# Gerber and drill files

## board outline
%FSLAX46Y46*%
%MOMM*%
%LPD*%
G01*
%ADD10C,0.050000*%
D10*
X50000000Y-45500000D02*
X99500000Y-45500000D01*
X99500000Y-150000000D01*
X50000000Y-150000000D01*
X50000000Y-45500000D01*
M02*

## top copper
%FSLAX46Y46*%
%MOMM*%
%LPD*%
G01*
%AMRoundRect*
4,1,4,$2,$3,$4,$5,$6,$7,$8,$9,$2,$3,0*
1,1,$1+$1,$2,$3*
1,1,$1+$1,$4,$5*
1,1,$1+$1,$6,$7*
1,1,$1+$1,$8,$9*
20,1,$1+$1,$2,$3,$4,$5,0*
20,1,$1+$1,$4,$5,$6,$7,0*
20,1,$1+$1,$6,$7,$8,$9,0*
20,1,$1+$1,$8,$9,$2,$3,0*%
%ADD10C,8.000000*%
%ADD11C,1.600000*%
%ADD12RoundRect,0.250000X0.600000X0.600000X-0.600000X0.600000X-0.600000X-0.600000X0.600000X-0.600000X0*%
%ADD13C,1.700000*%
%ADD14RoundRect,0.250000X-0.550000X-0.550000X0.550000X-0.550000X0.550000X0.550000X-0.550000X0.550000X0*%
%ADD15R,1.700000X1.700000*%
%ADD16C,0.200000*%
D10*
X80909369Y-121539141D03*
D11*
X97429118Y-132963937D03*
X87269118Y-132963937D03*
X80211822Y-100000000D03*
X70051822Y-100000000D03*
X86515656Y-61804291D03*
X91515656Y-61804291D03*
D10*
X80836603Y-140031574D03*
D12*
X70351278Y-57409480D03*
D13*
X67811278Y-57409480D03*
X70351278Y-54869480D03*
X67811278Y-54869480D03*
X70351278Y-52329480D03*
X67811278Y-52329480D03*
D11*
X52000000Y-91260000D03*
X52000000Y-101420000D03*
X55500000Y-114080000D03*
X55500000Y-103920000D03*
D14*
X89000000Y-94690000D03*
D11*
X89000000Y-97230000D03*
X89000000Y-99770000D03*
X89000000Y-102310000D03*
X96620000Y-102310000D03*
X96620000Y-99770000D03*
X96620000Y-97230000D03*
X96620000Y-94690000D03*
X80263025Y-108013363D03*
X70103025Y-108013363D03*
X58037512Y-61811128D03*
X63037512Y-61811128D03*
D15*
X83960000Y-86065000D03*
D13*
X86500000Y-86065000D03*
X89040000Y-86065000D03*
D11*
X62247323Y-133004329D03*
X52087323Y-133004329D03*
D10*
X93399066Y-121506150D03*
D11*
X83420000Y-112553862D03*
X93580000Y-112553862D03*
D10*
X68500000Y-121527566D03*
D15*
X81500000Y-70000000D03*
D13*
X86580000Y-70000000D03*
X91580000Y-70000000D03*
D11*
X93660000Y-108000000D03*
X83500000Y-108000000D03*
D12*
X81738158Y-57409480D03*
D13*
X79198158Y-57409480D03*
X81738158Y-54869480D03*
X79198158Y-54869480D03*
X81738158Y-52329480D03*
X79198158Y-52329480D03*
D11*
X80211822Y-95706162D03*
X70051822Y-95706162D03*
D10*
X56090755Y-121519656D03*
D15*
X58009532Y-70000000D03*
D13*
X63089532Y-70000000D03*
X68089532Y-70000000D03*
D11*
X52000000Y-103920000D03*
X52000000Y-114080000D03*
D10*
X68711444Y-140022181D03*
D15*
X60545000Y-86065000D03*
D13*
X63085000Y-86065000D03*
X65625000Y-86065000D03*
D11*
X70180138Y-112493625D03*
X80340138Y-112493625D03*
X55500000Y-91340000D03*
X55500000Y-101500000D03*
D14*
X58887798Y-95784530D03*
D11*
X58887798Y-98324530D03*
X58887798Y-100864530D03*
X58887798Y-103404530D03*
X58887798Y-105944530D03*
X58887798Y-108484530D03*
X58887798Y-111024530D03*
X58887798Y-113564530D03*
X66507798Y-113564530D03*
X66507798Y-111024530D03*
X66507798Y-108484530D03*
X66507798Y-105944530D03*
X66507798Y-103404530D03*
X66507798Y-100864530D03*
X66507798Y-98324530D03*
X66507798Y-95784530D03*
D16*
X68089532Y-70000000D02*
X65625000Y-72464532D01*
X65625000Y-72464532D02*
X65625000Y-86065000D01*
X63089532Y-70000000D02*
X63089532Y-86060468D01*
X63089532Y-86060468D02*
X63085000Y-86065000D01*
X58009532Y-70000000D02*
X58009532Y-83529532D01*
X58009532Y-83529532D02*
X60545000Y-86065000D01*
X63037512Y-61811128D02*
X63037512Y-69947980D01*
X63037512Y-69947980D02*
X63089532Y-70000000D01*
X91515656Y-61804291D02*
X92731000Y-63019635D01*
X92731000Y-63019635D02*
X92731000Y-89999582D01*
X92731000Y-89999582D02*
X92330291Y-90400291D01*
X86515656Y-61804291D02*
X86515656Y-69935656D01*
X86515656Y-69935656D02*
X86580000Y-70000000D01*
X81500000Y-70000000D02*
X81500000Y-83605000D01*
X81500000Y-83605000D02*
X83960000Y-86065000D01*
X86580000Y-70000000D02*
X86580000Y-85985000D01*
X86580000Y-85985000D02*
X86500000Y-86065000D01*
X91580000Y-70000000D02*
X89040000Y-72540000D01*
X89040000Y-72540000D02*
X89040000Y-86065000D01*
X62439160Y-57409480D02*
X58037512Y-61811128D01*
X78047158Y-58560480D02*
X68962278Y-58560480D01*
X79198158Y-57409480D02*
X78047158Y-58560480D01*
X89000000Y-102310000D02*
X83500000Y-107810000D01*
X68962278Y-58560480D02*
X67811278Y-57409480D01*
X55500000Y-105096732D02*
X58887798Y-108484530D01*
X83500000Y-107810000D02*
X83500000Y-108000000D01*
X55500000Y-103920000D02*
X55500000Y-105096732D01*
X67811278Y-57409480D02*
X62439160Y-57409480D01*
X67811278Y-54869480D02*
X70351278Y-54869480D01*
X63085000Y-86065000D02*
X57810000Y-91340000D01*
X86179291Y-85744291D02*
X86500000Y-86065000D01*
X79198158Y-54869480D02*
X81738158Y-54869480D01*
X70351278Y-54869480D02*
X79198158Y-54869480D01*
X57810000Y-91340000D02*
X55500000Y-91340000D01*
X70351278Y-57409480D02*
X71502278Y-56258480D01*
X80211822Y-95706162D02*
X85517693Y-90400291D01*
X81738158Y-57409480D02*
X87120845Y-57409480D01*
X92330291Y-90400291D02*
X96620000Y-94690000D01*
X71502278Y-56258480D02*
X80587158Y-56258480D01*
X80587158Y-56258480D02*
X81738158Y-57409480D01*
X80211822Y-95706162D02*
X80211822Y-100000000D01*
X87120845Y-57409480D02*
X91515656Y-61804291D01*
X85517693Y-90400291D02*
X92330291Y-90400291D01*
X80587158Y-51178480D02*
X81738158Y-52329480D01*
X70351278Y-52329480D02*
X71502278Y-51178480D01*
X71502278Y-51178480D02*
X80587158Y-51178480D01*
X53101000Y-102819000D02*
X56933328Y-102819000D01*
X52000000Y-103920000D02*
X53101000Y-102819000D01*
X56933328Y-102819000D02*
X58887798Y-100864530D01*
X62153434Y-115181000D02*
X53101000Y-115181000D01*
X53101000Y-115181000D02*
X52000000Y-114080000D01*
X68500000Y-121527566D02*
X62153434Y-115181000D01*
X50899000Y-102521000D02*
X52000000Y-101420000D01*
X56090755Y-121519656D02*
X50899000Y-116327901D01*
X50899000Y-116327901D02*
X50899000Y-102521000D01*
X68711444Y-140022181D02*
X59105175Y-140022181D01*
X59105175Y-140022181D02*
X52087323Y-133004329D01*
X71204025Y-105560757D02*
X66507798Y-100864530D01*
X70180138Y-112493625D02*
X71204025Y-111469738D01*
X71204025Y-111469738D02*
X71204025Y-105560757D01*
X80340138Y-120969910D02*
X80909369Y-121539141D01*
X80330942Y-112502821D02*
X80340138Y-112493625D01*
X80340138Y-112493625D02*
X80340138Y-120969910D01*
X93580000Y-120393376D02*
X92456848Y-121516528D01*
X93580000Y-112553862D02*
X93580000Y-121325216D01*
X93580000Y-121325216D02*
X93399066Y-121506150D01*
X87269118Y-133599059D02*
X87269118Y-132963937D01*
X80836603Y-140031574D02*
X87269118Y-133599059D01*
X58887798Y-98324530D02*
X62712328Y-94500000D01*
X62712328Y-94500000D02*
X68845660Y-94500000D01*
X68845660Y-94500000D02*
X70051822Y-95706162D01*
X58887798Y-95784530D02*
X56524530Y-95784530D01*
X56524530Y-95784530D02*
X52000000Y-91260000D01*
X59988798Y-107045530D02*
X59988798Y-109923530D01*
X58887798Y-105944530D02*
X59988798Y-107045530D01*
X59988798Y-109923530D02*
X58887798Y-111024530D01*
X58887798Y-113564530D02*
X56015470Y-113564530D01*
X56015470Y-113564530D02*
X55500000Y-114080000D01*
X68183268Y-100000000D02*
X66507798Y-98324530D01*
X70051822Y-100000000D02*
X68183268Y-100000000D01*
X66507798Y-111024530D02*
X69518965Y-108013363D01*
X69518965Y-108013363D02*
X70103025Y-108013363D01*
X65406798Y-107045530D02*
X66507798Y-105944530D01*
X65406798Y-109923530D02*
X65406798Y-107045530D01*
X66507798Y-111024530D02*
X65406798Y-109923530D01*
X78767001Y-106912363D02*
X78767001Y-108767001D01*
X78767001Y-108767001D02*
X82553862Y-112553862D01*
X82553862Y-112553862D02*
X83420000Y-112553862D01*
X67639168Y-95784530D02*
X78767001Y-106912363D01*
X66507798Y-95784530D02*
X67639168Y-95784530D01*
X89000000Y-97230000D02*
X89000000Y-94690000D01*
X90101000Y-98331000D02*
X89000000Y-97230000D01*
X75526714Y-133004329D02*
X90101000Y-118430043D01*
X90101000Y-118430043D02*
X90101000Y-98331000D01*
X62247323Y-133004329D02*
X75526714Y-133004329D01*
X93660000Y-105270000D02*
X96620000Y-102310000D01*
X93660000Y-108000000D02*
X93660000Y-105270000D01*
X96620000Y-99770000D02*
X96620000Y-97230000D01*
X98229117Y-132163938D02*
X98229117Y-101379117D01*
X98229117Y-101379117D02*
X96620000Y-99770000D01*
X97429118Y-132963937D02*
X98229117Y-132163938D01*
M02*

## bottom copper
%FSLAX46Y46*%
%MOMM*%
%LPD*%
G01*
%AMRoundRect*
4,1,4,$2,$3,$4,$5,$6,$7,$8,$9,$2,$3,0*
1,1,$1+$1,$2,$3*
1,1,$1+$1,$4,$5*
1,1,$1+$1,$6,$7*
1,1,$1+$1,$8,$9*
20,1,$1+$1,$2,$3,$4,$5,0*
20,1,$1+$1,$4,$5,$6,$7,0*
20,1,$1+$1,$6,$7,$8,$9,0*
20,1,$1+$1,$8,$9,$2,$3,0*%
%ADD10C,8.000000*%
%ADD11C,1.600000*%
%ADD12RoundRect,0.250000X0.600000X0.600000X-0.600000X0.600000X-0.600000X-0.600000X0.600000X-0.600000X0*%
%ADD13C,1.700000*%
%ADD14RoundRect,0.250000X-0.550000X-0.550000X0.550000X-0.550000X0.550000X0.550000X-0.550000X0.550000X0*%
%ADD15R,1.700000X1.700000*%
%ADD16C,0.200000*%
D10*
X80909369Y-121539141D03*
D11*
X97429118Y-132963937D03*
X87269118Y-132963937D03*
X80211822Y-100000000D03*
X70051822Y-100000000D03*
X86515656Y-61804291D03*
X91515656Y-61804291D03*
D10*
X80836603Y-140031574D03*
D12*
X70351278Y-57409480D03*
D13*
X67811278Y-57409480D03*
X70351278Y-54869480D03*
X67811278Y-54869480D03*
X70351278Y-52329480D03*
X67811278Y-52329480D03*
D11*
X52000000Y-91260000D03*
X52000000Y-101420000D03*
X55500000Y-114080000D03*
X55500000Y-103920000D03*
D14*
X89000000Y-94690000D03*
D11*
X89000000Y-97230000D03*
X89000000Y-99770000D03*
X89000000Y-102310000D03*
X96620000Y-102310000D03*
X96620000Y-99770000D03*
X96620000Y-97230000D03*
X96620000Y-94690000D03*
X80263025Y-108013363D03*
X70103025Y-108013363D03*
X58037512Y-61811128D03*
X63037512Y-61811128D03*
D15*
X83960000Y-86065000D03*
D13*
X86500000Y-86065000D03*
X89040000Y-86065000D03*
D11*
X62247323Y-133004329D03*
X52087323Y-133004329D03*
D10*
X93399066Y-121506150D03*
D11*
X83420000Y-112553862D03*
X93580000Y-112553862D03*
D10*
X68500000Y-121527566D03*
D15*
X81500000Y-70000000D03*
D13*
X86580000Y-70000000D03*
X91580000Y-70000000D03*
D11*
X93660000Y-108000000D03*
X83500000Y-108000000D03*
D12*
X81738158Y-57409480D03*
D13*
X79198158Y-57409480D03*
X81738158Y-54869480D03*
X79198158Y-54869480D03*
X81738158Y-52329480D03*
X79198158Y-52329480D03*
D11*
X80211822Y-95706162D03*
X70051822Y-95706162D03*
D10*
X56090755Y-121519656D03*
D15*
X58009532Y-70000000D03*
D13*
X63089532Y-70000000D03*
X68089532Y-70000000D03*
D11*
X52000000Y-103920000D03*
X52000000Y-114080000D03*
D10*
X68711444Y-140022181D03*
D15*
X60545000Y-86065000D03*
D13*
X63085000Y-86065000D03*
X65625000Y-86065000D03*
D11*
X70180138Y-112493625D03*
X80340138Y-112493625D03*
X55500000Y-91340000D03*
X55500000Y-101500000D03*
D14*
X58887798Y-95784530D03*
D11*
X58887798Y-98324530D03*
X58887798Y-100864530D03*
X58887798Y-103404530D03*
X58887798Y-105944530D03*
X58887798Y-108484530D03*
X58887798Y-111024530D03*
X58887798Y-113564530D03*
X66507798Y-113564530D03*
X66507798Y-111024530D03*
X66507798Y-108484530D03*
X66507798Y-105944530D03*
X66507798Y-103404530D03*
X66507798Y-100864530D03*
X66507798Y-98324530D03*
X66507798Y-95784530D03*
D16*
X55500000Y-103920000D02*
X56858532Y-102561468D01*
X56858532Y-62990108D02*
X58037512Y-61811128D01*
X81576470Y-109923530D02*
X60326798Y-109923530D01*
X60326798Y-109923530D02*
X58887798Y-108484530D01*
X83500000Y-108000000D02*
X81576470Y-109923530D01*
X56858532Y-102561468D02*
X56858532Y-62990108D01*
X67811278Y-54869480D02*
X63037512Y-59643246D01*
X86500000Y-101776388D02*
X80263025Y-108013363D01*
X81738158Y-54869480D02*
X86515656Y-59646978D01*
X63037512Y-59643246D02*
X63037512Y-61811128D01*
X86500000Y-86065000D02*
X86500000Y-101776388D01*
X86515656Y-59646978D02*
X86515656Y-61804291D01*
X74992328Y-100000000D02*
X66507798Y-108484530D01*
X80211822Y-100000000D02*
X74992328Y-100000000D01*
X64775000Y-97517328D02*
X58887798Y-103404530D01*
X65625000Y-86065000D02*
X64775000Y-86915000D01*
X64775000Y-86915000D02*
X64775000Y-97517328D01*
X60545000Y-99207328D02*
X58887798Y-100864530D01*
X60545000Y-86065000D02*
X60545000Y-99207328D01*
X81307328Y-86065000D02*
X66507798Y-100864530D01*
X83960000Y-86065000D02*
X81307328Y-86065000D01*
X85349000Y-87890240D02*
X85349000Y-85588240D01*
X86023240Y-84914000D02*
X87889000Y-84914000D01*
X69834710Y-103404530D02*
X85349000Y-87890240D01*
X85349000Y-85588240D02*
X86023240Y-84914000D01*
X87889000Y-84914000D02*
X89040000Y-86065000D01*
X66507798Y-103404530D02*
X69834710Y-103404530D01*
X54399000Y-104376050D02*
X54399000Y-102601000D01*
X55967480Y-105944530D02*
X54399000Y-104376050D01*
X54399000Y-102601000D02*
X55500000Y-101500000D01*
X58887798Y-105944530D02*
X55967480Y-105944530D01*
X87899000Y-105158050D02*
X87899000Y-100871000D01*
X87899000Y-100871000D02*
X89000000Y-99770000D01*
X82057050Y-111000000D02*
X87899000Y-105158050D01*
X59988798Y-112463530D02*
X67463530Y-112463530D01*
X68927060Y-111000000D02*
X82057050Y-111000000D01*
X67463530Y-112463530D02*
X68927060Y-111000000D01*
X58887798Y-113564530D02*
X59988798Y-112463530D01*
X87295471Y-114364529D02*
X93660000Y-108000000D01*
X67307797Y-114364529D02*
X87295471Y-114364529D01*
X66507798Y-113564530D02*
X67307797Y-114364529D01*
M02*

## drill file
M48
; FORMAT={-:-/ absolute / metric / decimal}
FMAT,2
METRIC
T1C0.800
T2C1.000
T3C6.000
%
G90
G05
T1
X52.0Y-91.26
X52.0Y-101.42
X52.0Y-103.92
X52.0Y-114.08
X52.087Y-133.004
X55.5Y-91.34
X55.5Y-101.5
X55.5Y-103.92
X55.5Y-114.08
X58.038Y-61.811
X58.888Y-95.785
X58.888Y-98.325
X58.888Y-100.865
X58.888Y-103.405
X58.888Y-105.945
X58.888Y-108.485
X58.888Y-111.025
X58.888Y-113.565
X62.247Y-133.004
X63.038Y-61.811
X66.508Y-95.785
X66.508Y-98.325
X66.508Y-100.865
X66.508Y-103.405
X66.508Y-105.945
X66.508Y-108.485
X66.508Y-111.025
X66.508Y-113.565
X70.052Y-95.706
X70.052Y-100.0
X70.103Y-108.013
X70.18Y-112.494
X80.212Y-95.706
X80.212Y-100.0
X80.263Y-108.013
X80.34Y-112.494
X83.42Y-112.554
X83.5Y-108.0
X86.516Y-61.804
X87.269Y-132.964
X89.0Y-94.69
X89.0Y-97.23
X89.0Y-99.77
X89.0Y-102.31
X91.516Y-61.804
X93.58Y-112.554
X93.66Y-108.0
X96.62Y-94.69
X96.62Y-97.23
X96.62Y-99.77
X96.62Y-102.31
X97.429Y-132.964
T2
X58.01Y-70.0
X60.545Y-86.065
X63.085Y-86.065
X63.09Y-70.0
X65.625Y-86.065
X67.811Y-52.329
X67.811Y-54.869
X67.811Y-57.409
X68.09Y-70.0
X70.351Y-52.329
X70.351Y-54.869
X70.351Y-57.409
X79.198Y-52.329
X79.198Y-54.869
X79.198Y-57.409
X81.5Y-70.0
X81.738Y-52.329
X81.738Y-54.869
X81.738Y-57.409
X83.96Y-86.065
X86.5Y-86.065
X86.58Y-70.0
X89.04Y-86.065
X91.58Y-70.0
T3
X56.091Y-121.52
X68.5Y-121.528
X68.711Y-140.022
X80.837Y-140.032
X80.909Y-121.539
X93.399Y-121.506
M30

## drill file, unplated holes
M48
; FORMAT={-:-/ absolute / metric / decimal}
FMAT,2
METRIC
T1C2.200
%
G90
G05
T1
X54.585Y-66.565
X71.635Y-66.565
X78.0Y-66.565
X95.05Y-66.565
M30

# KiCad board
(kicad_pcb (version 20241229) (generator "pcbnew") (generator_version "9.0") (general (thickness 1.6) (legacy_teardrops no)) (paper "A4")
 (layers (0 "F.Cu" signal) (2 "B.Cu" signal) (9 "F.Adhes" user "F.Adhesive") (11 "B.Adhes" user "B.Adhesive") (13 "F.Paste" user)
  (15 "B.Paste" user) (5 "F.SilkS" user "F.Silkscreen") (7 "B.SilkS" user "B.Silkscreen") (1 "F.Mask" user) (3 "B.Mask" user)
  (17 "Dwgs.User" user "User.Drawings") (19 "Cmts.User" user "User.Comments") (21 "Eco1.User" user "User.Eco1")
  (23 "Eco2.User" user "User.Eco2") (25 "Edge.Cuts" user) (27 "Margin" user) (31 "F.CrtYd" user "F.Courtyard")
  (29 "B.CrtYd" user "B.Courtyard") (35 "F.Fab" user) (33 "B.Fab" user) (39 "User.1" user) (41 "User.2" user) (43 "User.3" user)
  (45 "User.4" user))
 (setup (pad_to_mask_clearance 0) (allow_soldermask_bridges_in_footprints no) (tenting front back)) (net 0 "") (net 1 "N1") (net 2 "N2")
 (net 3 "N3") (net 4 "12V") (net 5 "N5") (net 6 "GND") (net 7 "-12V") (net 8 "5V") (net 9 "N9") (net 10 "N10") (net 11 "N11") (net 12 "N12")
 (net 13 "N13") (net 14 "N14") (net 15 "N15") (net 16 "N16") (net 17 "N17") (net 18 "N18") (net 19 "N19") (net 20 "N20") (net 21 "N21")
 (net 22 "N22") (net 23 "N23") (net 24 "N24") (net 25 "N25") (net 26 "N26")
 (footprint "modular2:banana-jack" (layer "F.Cu") (at 80.909369 121.514203)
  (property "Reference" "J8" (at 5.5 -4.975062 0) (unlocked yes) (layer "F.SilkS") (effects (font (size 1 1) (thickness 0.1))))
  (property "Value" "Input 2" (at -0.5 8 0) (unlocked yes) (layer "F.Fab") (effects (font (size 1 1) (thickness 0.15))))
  (pad "1" thru_hole circle (at 0 0.024938) (size 8 8) (drill 6) (layers "*.Cu" "*.Mask") (remove_unused_layers no) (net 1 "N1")))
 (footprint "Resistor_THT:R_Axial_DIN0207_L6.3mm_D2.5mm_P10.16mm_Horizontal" (layer "F.Cu") (at 97.429118 132.963937 180)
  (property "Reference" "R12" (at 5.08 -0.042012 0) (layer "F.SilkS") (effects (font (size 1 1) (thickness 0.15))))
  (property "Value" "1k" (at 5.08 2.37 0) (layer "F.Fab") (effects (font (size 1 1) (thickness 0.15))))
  (pad "1" thru_hole circle (at 0 0 180) (size 1.6 1.6) (drill 0.8) (layers "*.Cu" "*.Mask") (remove_unused_layers no) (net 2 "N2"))
  (pad "2" thru_hole circle (at 10.16 0 180) (size 1.6 1.6) (drill 0.8) (layers "*.Cu" "*.Mask") (remove_unused_layers no) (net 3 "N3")))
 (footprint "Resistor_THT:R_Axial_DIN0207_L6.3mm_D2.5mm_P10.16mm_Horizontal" (layer "F.Cu") (at 80.211822 100 180)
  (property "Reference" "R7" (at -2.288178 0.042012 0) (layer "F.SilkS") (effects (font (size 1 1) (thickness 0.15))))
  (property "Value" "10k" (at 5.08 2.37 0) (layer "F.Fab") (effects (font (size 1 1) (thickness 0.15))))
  (pad "1" thru_hole circle (at 0 0 180) (size 1.6 1.6) (drill 0.8) (layers "*.Cu" "*.Mask") (remove_unused_layers no) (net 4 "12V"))
  (pad "2" thru_hole circle (at 10.16 0 180) (size 1.6 1.6) (drill 0.8) (layers "*.Cu" "*.Mask") (remove_unused_layers no) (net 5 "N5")))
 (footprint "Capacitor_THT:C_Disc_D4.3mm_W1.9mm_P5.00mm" (layer "F.Cu") (at 86.515656 61.804291)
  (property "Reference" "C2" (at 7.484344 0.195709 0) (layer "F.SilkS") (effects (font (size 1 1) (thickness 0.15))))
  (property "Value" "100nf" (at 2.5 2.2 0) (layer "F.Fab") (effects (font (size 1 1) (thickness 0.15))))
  (pad "1" thru_hole circle (at 0 0) (size 1.6 1.6) (drill 0.8) (layers "*.Cu" "*.Mask") (remove_unused_layers no) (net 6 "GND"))
  (pad "2" thru_hole circle (at 5 0) (size 1.6 1.6) (drill 0.8) (layers "*.Cu" "*.Mask") (remove_unused_layers no) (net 4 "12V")))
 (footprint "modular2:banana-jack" (layer "F.Cu") (at 80.836603 140.006636)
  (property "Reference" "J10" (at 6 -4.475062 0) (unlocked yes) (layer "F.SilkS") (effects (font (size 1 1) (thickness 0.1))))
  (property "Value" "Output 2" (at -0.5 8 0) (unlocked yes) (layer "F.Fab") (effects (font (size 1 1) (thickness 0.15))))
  (pad "1" thru_hole circle (at 0 0.024938) (size 8 8) (drill 6) (layers "*.Cu" "*.Mask") (remove_unused_layers no) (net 3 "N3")))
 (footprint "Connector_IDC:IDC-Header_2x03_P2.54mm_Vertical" (layer "F.Cu") (at 70.351278 57.40948 180)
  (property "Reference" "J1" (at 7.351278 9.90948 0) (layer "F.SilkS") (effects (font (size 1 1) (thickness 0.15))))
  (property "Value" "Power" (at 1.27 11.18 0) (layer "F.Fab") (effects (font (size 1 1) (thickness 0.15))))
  (pad "1" thru_hole roundrect (at 0 0 180) (size 1.7 1.7) (drill 1) (layers "*.Cu" "*.Mask") (remove_unused_layers no)
   (roundrect_rratio 0.147059) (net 4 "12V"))
  (pad "2" thru_hole circle (at 2.54 0 180) (size 1.7 1.7) (drill 1) (layers "*.Cu" "*.Mask") (remove_unused_layers no) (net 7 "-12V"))
  (pad "3" thru_hole circle (at 0 2.54 180) (size 1.7 1.7) (drill 1) (layers "*.Cu" "*.Mask") (remove_unused_layers no) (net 6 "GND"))
  (pad "4" thru_hole circle (at 2.54 2.54 180) (size 1.7 1.7) (drill 1) (layers "*.Cu" "*.Mask") (remove_unused_layers no) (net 6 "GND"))
  (pad "5" thru_hole circle (at 0 5.08 180) (size 1.7 1.7) (drill 1) (layers "*.Cu" "*.Mask") (remove_unused_layers no) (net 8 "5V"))
  (pad "6" thru_hole circle (at 2.54 5.08 180) (size 1.7 1.7) (drill 1) (layers "*.Cu" "*.Mask") (remove_unused_layers no) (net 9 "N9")))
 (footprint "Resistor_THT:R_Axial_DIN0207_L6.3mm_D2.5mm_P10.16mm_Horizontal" (layer "F.Cu") (at 52 91.26 -90)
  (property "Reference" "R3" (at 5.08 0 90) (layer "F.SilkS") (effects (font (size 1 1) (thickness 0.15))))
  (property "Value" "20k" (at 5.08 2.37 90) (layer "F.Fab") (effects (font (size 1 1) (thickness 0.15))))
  (pad "1" thru_hole circle (at 0 0 270) (size 1.6 1.6) (drill 0.8) (layers "*.Cu" "*.Mask") (remove_unused_layers no) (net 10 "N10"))
  (pad "2" thru_hole circle (at 10.16 0 270) (size 1.6 1.6) (drill 0.8) (layers "*.Cu" "*.Mask") (remove_unused_layers no) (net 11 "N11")))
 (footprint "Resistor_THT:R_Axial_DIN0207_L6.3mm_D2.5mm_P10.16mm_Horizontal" (layer "F.Cu") (at 55.5 114.08 90)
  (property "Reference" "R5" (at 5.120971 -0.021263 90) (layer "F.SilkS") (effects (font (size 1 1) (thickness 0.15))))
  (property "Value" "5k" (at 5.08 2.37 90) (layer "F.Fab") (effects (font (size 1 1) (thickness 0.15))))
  (pad "1" thru_hole circle (at 0 0 90) (size 1.6 1.6) (drill 0.8) (layers "*.Cu" "*.Mask") (remove_unused_layers no) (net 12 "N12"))
  (pad "2" thru_hole circle (at 10.16 0 90) (size 1.6 1.6) (drill 0.8) (layers "*.Cu" "*.Mask") (remove_unused_layers no) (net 7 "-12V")))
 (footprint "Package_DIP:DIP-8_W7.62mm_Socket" (layer "F.Cu") (at 89 94.69)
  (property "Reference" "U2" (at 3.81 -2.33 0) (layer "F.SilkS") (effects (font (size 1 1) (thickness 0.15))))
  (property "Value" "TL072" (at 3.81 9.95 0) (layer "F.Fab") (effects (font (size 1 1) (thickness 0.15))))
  (pad "1" thru_hole roundrect (at 0 0) (size 1.6 1.6) (drill 0.8) (layers "*.Cu" "*.Mask") (remove_unused_layers no)
   (roundrect_rratio 0.15625) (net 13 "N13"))
  (pad "2" thru_hole circle (at 0 2.54) (size 1.6 1.6) (drill 0.8) (layers "*.Cu" "*.Mask") (remove_unused_layers no) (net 13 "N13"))
  (pad "3" thru_hole circle (at 0 5.08) (size 1.6 1.6) (drill 0.8) (layers "*.Cu" "*.Mask") (remove_unused_layers no) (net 12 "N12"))
  (pad "4" thru_hole circle (at 0 7.62) (size 1.6 1.6) (drill 0.8) (layers "*.Cu" "*.Mask") (remove_unused_layers no) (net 7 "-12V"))
  (pad "5" thru_hole circle (at 7.62 7.62) (size 1.6 1.6) (drill 0.8) (layers "*.Cu" "*.Mask") (remove_unused_layers no) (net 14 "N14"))
  (pad "6" thru_hole circle (at 7.62 5.08) (size 1.6 1.6) (drill 0.8) (layers "*.Cu" "*.Mask") (remove_unused_layers no) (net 2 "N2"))
  (pad "7" thru_hole circle (at 7.62 2.54) (size 1.6 1.6) (drill 0.8) (layers "*.Cu" "*.Mask") (remove_unused_layers no) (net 2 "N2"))
  (pad "8" thru_hole circle (at 7.62 0) (size 1.6 1.6) (drill 0.8) (layers "*.Cu" "*.Mask") (remove_unused_layers no) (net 4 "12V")))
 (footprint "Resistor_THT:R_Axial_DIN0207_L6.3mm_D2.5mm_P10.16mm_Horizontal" (layer "F.Cu") (at 80.263025 108.013363 180)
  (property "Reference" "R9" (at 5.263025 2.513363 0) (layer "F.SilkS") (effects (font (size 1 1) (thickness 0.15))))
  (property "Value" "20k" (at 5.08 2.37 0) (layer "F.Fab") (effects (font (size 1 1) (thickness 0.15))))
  (pad "1" thru_hole circle (at 0 0 180) (size 1.6 1.6) (drill 0.8) (layers "*.Cu" "*.Mask") (remove_unused_layers no) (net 6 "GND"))
  (pad "2" thru_hole circle (at 10.16 0 180) (size 1.6 1.6) (drill 0.8) (layers "*.Cu" "*.Mask") (remove_unused_layers no) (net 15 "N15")))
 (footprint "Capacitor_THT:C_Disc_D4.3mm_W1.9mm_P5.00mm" (layer "F.Cu") (at 58.037512 61.811128)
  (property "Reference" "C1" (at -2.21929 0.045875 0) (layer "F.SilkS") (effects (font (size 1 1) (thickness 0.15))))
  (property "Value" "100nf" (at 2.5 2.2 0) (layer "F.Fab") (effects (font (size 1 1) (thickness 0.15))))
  (pad "1" thru_hole circle (at 0 0) (size 1.6 1.6) (drill 0.8) (layers "*.Cu" "*.Mask") (remove_unused_layers no) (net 7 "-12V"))
  (pad "2" thru_hole circle (at 5 0) (size 1.6 1.6) (drill 0.8) (layers "*.Cu" "*.Mask") (remove_unused_layers no) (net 6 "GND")))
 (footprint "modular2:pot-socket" (layer "F.Cu") (at 85.5 78.065)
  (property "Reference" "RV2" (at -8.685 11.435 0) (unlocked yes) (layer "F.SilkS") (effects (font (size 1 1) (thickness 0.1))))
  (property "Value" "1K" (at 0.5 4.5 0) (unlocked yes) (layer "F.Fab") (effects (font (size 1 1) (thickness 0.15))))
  (pad "" np_thru_hole circle (at -7.5 -11.5) (size 2.2 2.2) (drill 2.2) (layers "*.Cu" "*.Mask"))
  (pad "" np_thru_hole circle (at 9.55 -11.5) (size 2.2 2.2) (drill 2.2) (layers "*.Cu" "*.Mask"))
  (pad "1" thru_hole rect (at -1.54 8 90) (size 1.7 1.7) (drill 1) (layers "*.Cu" "*.Mask") (remove_unused_layers no) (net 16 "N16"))
  (pad "2" thru_hole circle (at 1 8 90) (size 1.7 1.7) (drill 1) (layers "*.Cu" "*.Mask") (remove_unused_layers no) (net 6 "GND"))
  (pad "3" thru_hole circle (at 3.54 8 90) (size 1.7 1.7) (drill 1) (layers "*.Cu" "*.Mask") (remove_unused_layers no) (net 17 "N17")))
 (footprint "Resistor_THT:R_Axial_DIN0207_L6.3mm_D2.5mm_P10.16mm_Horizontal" (layer "F.Cu") (at 62.247323 133.004329 180)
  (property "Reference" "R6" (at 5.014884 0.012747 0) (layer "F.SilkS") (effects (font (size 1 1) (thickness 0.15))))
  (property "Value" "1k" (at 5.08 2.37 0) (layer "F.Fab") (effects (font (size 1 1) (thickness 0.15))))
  (pad "1" thru_hole circle (at 0 0 180) (size 1.6 1.6) (drill 0.8) (layers "*.Cu" "*.Mask") (remove_unused_layers no) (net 13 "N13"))
  (pad "2" thru_hole circle (at 10.16 0 180) (size 1.6 1.6) (drill 0.8) (layers "*.Cu" "*.Mask") (remove_unused_layers no) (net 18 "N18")))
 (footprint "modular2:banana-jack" (layer "F.Cu") (at 93.399066 121.481212)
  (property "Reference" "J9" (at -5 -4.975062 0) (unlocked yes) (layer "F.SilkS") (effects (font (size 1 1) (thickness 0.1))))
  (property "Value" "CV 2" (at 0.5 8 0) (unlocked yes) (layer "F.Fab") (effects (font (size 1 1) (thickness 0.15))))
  (pad "1" thru_hole circle (at 0 0.024938) (size 8 8) (drill 6) (layers "*.Cu" "*.Mask") (remove_unused_layers no) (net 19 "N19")))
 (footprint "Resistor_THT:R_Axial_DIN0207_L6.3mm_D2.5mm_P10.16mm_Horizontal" (layer "F.Cu") (at 83.42 112.553862)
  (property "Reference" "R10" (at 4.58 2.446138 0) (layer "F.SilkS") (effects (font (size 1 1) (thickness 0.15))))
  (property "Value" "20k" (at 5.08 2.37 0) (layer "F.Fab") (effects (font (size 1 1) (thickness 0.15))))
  (pad "1" thru_hole circle (at 0 0) (size 1.6 1.6) (drill 0.8) (layers "*.Cu" "*.Mask") (remove_unused_layers no) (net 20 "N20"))
  (pad "2" thru_hole circle (at 10.16 0) (size 1.6 1.6) (drill 0.8) (layers "*.Cu" "*.Mask") (remove_unused_layers no) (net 19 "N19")))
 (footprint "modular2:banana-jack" (layer "F.Cu") (at 68.5 121.502628)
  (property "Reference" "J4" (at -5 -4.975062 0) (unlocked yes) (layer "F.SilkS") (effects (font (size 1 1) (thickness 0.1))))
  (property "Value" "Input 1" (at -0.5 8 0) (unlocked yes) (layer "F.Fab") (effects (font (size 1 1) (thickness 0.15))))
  (pad "1" thru_hole circle (at 0 0.024938) (size 8 8) (drill 6) (layers "*.Cu" "*.Mask") (remove_unused_layers no) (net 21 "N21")))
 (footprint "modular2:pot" (layer "F.Cu") (at 86.58 73)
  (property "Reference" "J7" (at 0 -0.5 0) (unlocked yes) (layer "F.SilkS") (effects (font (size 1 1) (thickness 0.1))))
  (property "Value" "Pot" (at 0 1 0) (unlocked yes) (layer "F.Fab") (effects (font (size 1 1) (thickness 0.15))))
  (pad "1" thru_hole rect (at -5.08 -3 90) (size 1.7 1.7) (drill 1) (layers "*.Cu" "*.Mask") (remove_unused_layers no) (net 16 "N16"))
  (pad "2" thru_hole circle (at 0 -3 90) (size 1.7 1.7) (drill 1) (layers "*.Cu" "*.Mask") (remove_unused_layers no) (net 6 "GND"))
  (pad "3" thru_hole circle (at 5 -3 90) (size 1.7 1.7) (drill 1) (layers "*.Cu" "*.Mask") (remove_unused_layers no) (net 17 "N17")))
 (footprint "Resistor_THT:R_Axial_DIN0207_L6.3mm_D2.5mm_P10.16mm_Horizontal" (layer "F.Cu") (at 93.66 108 180)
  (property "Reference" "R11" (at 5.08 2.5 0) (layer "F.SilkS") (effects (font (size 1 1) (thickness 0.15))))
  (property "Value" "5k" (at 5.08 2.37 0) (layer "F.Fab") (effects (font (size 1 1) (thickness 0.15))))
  (pad "1" thru_hole circle (at 0 0 180) (size 1.6 1.6) (drill 0.8) (layers "*.Cu" "*.Mask") (remove_unused_layers no) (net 14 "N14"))
  (pad "2" thru_hole circle (at 10.16 0 180) (size 1.6 1.6) (drill 0.8) (layers "*.Cu" "*.Mask") (remove_unused_layers no) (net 7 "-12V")))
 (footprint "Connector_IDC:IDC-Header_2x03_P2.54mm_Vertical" (layer "F.Cu") (at 81.738158 57.40948 180)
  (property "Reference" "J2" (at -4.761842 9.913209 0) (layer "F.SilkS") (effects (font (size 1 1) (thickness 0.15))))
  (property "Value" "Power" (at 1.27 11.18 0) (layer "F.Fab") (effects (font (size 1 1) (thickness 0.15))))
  (pad "1" thru_hole roundrect (at 0 0 180) (size 1.7 1.7) (drill 1) (layers "*.Cu" "*.Mask") (remove_unused_layers no)
   (roundrect_rratio 0.147059) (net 4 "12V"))
  (pad "2" thru_hole circle (at 2.54 0 180) (size 1.7 1.7) (drill 1) (layers "*.Cu" "*.Mask") (remove_unused_layers no) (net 7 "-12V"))
  (pad "3" thru_hole circle (at 0 2.54 180) (size 1.7 1.7) (drill 1) (layers "*.Cu" "*.Mask") (remove_unused_layers no) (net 6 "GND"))
  (pad "4" thru_hole circle (at 2.54 2.54 180) (size 1.7 1.7) (drill 1) (layers "*.Cu" "*.Mask") (remove_unused_layers no) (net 6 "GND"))
  (pad "5" thru_hole circle (at 0 5.08 180) (size 1.7 1.7) (drill 1) (layers "*.Cu" "*.Mask") (remove_unused_layers no) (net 8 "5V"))
  (pad "6" thru_hole circle (at 2.54 5.08 180) (size 1.7 1.7) (drill 1) (layers "*.Cu" "*.Mask") (remove_unused_layers no) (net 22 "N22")))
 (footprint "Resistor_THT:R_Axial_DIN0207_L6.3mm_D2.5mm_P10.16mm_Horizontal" (layer "F.Cu") (at 80.211822 95.706162 180)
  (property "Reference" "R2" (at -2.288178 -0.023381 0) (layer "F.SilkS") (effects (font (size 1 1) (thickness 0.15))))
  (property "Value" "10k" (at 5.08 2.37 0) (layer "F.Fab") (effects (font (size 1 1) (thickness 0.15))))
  (pad "1" thru_hole circle (at 0 0 180) (size 1.6 1.6) (drill 0.8) (layers "*.Cu" "*.Mask") (remove_unused_layers no) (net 4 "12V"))
  (pad "2" thru_hole circle (at 10.16 0 180) (size 1.6 1.6) (drill 0.8) (layers "*.Cu" "*.Mask") (remove_unused_layers no) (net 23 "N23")))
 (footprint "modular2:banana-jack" (layer "F.Cu") (at 56.090755 121.494718)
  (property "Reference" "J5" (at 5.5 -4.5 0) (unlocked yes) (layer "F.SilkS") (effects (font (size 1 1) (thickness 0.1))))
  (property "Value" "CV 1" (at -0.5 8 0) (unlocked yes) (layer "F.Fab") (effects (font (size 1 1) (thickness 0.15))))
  (pad "1" thru_hole circle (at 0 0.024938) (size 8 8) (drill 6) (layers "*.Cu" "*.Mask") (remove_unused_layers no) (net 11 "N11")))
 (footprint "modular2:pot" (layer "F.Cu") (at 63.089532 73)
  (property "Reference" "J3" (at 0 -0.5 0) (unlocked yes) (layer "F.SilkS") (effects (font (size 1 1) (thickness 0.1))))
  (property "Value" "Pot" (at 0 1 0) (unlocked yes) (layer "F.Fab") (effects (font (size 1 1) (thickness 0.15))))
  (pad "1" thru_hole rect (at -5.08 -3 90) (size 1.7 1.7) (drill 1) (layers "*.Cu" "*.Mask") (remove_unused_layers no) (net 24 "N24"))
  (pad "2" thru_hole circle (at 0 -3 90) (size 1.7 1.7) (drill 1) (layers "*.Cu" "*.Mask") (remove_unused_layers no) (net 6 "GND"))
  (pad "3" thru_hole circle (at 5 -3 90) (size 1.7 1.7) (drill 1) (layers "*.Cu" "*.Mask") (remove_unused_layers no) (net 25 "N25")))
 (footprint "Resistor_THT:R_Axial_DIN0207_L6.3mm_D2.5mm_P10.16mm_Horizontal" (layer "F.Cu") (at 52 103.92 -90)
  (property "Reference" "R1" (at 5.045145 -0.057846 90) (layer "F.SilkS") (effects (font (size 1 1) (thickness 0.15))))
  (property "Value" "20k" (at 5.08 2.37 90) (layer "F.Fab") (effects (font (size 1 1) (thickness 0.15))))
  (pad "1" thru_hole circle (at 0 0 270) (size 1.6 1.6) (drill 0.8) (layers "*.Cu" "*.Mask") (remove_unused_layers no) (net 24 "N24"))
  (pad "2" thru_hole circle (at 10.16 0 270) (size 1.6 1.6) (drill 0.8) (layers "*.Cu" "*.Mask") (remove_unused_layers no) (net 21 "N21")))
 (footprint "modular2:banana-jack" (layer "F.Cu") (at 68.711444 139.997243)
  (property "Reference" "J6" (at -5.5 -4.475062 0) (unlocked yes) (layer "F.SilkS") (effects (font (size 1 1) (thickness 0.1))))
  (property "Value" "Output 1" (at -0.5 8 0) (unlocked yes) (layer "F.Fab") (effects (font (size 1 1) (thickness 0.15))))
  (pad "1" thru_hole circle (at 0 0.024938) (size 8 8) (drill 6) (layers "*.Cu" "*.Mask") (remove_unused_layers no) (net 18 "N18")))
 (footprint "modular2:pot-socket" (layer "F.Cu") (at 62.085 78.065)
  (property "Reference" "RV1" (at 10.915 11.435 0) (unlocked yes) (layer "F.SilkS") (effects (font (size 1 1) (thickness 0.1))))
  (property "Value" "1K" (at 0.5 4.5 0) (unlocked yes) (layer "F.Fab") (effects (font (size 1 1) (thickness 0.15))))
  (pad "" np_thru_hole circle (at -7.5 -11.5) (size 2.2 2.2) (drill 2.2) (layers "*.Cu" "*.Mask"))
  (pad "" np_thru_hole circle (at 9.55 -11.5) (size 2.2 2.2) (drill 2.2) (layers "*.Cu" "*.Mask"))
  (pad "1" thru_hole rect (at -1.54 8 90) (size 1.7 1.7) (drill 1) (layers "*.Cu" "*.Mask") (remove_unused_layers no) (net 24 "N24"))
  (pad "2" thru_hole circle (at 1 8 90) (size 1.7 1.7) (drill 1) (layers "*.Cu" "*.Mask") (remove_unused_layers no) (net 6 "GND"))
  (pad "3" thru_hole circle (at 3.54 8 90) (size 1.7 1.7) (drill 1) (layers "*.Cu" "*.Mask") (remove_unused_layers no) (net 25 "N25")))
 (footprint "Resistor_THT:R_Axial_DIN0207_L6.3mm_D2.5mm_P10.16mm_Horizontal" (layer "F.Cu") (at 70.180138 112.493625)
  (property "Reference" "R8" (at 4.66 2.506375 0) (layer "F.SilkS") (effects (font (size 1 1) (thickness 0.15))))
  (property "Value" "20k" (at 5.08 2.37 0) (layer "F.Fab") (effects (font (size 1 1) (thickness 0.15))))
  (pad "1" thru_hole circle (at 0 0) (size 1.6 1.6) (drill 0.8) (layers "*.Cu" "*.Mask") (remove_unused_layers no) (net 16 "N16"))
  (pad "2" thru_hole circle (at 10.16 0) (size 1.6 1.6) (drill 0.8) (layers "*.Cu" "*.Mask") (remove_unused_layers no) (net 1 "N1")))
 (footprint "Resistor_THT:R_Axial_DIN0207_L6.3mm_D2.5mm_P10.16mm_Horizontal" (layer "F.Cu") (at 55.5 91.34 -90)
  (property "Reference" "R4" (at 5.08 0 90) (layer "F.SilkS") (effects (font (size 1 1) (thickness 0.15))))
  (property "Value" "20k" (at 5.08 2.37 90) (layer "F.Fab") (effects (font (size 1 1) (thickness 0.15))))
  (pad "1" thru_hole circle (at 0 0 270) (size 1.6 1.6) (drill 0.8) (layers "*.Cu" "*.Mask") (remove_unused_layers no) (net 6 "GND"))
  (pad "2" thru_hole circle (at 10.16 0 270) (size 1.6 1.6) (drill 0.8) (layers "*.Cu" "*.Mask") (remove_unused_layers no) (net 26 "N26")))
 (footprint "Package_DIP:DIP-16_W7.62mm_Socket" (layer "F.Cu") (at 58.887798 95.78453)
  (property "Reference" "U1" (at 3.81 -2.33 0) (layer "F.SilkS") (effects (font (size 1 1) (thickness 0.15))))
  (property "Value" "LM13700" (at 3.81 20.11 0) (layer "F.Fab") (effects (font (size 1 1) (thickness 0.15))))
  (pad "1" thru_hole roundrect (at 0 0) (size 1.6 1.6) (drill 0.8) (layers "*.Cu" "*.Mask") (remove_unused_layers no)
   (roundrect_rratio 0.15625) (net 10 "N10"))
  (pad "2" thru_hole circle (at 0 2.54) (size 1.6 1.6) (drill 0.8) (layers "*.Cu" "*.Mask") (remove_unused_layers no) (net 23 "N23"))
  (pad "3" thru_hole circle (at 0 5.08) (size 1.6 1.6) (drill 0.8) (layers "*.Cu" "*.Mask") (remove_unused_layers no) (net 24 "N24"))
  (pad "4" thru_hole circle (at 0 7.62) (size 1.6 1.6) (drill 0.8) (layers "*.Cu" "*.Mask") (remove_unused_layers no) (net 25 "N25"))
  (pad "5" thru_hole circle (at 0 10.16) (size 1.6 1.6) (drill 0.8) (layers "*.Cu" "*.Mask") (remove_unused_layers no) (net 26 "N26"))
  (pad "6" thru_hole circle (at 0 12.7) (size 1.6 1.6) (drill 0.8) (layers "*.Cu" "*.Mask") (remove_unused_layers no) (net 7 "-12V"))
  (pad "7" thru_hole circle (at 0 15.24) (size 1.6 1.6) (drill 0.8) (layers "*.Cu" "*.Mask") (remove_unused_layers no) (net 26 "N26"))
  (pad "8" thru_hole circle (at 0 17.78) (size 1.6 1.6) (drill 0.8) (layers "*.Cu" "*.Mask") (remove_unused_layers no) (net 12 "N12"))
  (pad "9" thru_hole circle (at 7.62 17.78) (size 1.6 1.6) (drill 0.8) (layers "*.Cu" "*.Mask") (remove_unused_layers no) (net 14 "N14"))
  (pad "10" thru_hole circle (at 7.62 15.24) (size 1.6 1.6) (drill 0.8) (layers "*.Cu" "*.Mask") (remove_unused_layers no) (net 15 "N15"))
  (pad "11" thru_hole circle (at 7.62 12.7) (size 1.6 1.6) (drill 0.8) (layers "*.Cu" "*.Mask") (remove_unused_layers no) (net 4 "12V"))
  (pad "12" thru_hole circle (at 7.62 10.16) (size 1.6 1.6) (drill 0.8) (layers "*.Cu" "*.Mask") (remove_unused_layers no) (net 15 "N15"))
  (pad "13" thru_hole circle (at 7.62 7.62) (size 1.6 1.6) (drill 0.8) (layers "*.Cu" "*.Mask") (remove_unused_layers no) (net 17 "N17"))
  (pad "14" thru_hole circle (at 7.62 5.08) (size 1.6 1.6) (drill 0.8) (layers "*.Cu" "*.Mask") (remove_unused_layers no) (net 16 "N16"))
  (pad "15" thru_hole circle (at 7.62 2.54) (size 1.6 1.6) (drill 0.8) (layers "*.Cu" "*.Mask") (remove_unused_layers no) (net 5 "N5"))
  (pad "16" thru_hole circle (at 7.62 0) (size 1.6 1.6) (drill 0.8) (layers "*.Cu" "*.Mask") (remove_unused_layers no) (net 20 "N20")))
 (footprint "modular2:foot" (layer "B.Cu") (at 56.59315 142.948114 180)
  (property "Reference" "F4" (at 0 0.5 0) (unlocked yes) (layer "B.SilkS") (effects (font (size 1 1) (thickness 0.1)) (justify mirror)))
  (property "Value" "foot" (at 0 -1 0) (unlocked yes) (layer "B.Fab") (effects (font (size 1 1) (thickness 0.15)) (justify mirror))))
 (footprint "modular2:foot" (layer "B.Cu") (at 92.94531 142.941798 180)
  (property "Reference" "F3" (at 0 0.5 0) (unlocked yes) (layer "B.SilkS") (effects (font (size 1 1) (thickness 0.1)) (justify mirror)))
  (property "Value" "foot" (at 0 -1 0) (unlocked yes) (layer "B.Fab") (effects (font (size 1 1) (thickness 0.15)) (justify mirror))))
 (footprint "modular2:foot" (layer "B.Cu") (at 56.600318 52.099806 180)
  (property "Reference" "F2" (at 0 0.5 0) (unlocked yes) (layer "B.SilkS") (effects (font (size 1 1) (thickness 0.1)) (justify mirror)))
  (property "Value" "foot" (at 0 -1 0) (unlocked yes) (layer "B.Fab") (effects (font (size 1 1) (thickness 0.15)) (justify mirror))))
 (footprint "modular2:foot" (layer "B.Cu") (at 92.943332 52.071217 180)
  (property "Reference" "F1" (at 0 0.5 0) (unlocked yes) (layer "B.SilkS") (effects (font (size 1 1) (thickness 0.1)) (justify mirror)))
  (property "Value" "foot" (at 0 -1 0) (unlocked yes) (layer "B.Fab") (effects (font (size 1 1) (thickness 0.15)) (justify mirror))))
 (gr_rect (start 50 45.5) (end 99.5 150) (stroke (width 0.05) (type default)) (fill no) (layer "Edge.Cuts"))
 (segment (start 62.43916 57.40948) (end 58.037512 61.811128) (width 0.2) (layer "F.Cu") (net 7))
 (segment (start 78.047158 58.56048) (end 68.962278 58.56048) (width 0.2) (layer "F.Cu") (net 7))
 (segment (start 79.198158 57.40948) (end 78.047158 58.56048) (width 0.2) (layer "F.Cu") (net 7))
 (segment (start 89 102.31) (end 83.5 107.81) (width 0.2) (layer "F.Cu") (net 7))
 (segment (start 68.962278 58.56048) (end 67.811278 57.40948) (width 0.2) (layer "F.Cu") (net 7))
 (segment (start 55.5 105.096732) (end 58.887798 108.48453) (width 0.2) (layer "F.Cu") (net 7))
 (segment (start 83.5 107.81) (end 83.5 108) (width 0.2) (layer "F.Cu") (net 7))
 (segment (start 55.5 103.92) (end 55.5 105.096732) (width 0.2) (layer "F.Cu") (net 7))
 (segment (start 67.811278 57.40948) (end 62.43916 57.40948) (width 0.2) (layer "F.Cu") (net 7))
 (segment (start 55.5 103.92) (end 56.858532 102.561468) (width 0.2) (layer "B.Cu") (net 7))
 (segment (start 56.858532 62.990108) (end 58.037512 61.811128) (width 0.2) (layer "B.Cu") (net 7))
 (segment (start 81.57647 109.92353) (end 60.326798 109.92353) (width 0.2) (layer "B.Cu") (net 7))
 (segment (start 60.326798 109.92353) (end 58.887798 108.48453) (width 0.2) (layer "B.Cu") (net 7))
 (segment (start 83.5 108) (end 81.57647 109.92353) (width 0.2) (layer "B.Cu") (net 7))
 (segment (start 56.858532 102.561468) (end 56.858532 62.990108) (width 0.2) (layer "B.Cu") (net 7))
 (segment (start 67.811278 54.86948) (end 70.351278 54.86948) (width 0.2) (layer "F.Cu") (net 6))
 (segment (start 63.089532 86.060468) (end 63.085 86.065) (width 0.2) (layer "F.Cu") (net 6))
 (segment (start 63.037512 61.811128) (end 63.037512 69.94798) (width 0.2) (layer "F.Cu") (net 6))
 (segment (start 86.58 85.985) (end 86.5 86.065) (width 0.2) (layer "F.Cu") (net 6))
 (segment (start 63.085 86.065) (end 57.81 91.34) (width 0.2) (layer "F.Cu") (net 6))
 (segment (start 86.179291 85.744291) (end 86.5 86.065) (width 0.2) (layer "F.Cu") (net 6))
 (segment (start 79.198158 54.86948) (end 81.738158 54.86948) (width 0.2) (layer "F.Cu") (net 6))
 (segment (start 63.037512 69.94798) (end 63.089532 70) (width 0.2) (layer "F.Cu") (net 6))
 (segment (start 70.351278 54.86948) (end 79.198158 54.86948) (width 0.2) (layer "F.Cu") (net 6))
 (segment (start 86.515656 69.935656) (end 86.58 70) (width 0.2) (layer "F.Cu") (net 6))
 (segment (start 57.81 91.34) (end 55.5 91.34) (width 0.2) (layer "F.Cu") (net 6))
 (segment (start 86.58 70) (end 86.58 85.985) (width 0.2) (layer "F.Cu") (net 6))
 (segment (start 63.089532 70) (end 63.089532 86.060468) (width 0.2) (layer "F.Cu") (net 6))
 (segment (start 86.515656 61.804291) (end 86.515656 69.935656) (width 0.2) (layer "F.Cu") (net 6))
 (segment (start 67.811278 54.86948) (end 63.037512 59.643246) (width 0.2) (layer "B.Cu") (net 6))
 (segment (start 86.5 101.776388) (end 80.263025 108.013363) (width 0.2) (layer "B.Cu") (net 6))
 (segment (start 81.738158 54.86948) (end 86.515656 59.646978) (width 0.2) (layer "B.Cu") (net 6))
 (segment (start 63.037512 59.643246) (end 63.037512 61.811128) (width 0.2) (layer "B.Cu") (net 6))
 (segment (start 86.5 86.065) (end 86.5 101.776388) (width 0.2) (layer "B.Cu") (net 6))
 (segment (start 86.515656 59.646978) (end 86.515656 61.804291) (width 0.2) (layer "B.Cu") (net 6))
 (segment (start 70.351278 57.40948) (end 71.502278 56.25848) (width 0.2) (layer "F.Cu") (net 4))
 (segment (start 80.211822 95.706162) (end 85.517693 90.400291) (width 0.2) (layer "F.Cu") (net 4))
 (segment (start 92.731 63.019635) (end 92.731 89.999582) (width 0.2) (layer "F.Cu") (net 4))
 (segment (start 81.738158 57.40948) (end 87.120845 57.40948) (width 0.2) (layer "F.Cu") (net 4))
 (segment (start 92.731 89.999582) (end 92.330291 90.400291) (width 0.2) (layer "F.Cu") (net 4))
 (segment (start 92.330291 90.400291) (end 96.62 94.69) (width 0.2) (layer "F.Cu") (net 4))
 (segment (start 71.502278 56.25848) (end 80.587158 56.25848) (width 0.2) (layer "F.Cu") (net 4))
 (segment (start 80.587158 56.25848) (end 81.738158 57.40948) (width 0.2) (layer "F.Cu") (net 4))
 (segment (start 80.211822 95.706162) (end 80.211822 100) (width 0.2) (layer "F.Cu") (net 4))
 (segment (start 87.120845 57.40948) (end 91.515656 61.804291) (width 0.2) (layer "F.Cu") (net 4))
 (segment (start 85.517693 90.400291) (end 92.330291 90.400291) (width 0.2) (layer "F.Cu") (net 4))
 (segment (start 91.515656 61.804291) (end 92.731 63.019635) (width 0.2) (layer "F.Cu") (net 4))
 (segment (start 74.992328 100) (end 66.507798 108.48453) (width 0.2) (layer "B.Cu") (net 4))
 (segment (start 80.211822 100) (end 74.992328 100) (width 0.2) (layer "B.Cu") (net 4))
 (segment (start 80.587158 51.17848) (end 81.738158 52.32948) (width 0.2) (layer "F.Cu") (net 8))
 (segment (start 70.351278 52.32948) (end 71.502278 51.17848) (width 0.2) (layer "F.Cu") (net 8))
 (segment (start 71.502278 51.17848) (end 80.587158 51.17848) (width 0.2) (layer "F.Cu") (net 8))
 (segment (start 65.625 72.464532) (end 65.625 86.065) (width 0.2) (layer "F.Cu") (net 25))
 (segment (start 68.089532 70) (end 65.625 72.464532) (width 0.2) (layer "F.Cu") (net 25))
 (segment (start 64.775 97.517328) (end 58.887798 103.40453) (width 0.2) (layer "B.Cu") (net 25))
 (segment (start 65.625 86.065) (end 64.775 86.915) (width 0.2) (layer "B.Cu") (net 25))
 (segment (start 64.775 86.915) (end 64.775 97.517328) (width 0.2) (layer "B.Cu") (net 25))
 (segment (start 53.101 102.819) (end 56.933328 102.819) (width 0.2) (layer "F.Cu") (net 24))
 (segment (start 52 103.92) (end 53.101 102.819) (width 0.2) (layer "F.Cu") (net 24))
 (segment (start 56.933328 102.819) (end 58.887798 100.86453) (width 0.2) (layer "F.Cu") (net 24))
 (segment (start 58.009532 83.529532) (end 60.545 86.065) (width 0.2) (layer "F.Cu") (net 24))
 (segment (start 58.009532 70) (end 58.009532 83.529532) (width 0.2) (layer "F.Cu") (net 24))
 (segment (start 60.545 99.207328) (end 58.887798 100.86453) (width 0.2) (layer "B.Cu") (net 24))
 (segment (start 60.545 86.065) (end 60.545 99.207328) (width 0.2) (layer "B.Cu") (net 24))
 (segment (start 62.153434 115.181) (end 53.101 115.181) (width 0.2) (layer "F.Cu") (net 21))
 (segment (start 53.101 115.181) (end 52 114.08) (width 0.2) (layer "F.Cu") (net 21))
 (segment (start 68.5 121.527566) (end 62.153434 115.181) (width 0.2) (layer "F.Cu") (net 21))
 (segment (start 50.899 102.521) (end 52 101.42) (width 0.2) (layer "F.Cu") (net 11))
 (segment (start 56.090755 121.519656) (end 50.899 116.327901) (width 0.2) (layer "F.Cu") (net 11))
 (segment (start 50.899 116.327901) (end 50.899 102.521) (width 0.2) (layer "F.Cu") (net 11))
 (segment (start 68.711444 140.022181) (end 59.105175 140.022181) (width 0.2) (layer "F.Cu") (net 18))
 (segment (start 59.105175 140.022181) (end 52.087323 133.004329) (width 0.2) (layer "F.Cu") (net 18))
 (segment (start 71.204025 105.560757) (end 66.507798 100.86453) (width 0.2) (layer "F.Cu") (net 16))
 (segment (start 81.5 83.605) (end 83.96 86.065) (width 0.2) (layer "F.Cu") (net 16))
 (segment (start 70.180138 112.493625) (end 71.204025 111.469738) (width 0.2) (layer "F.Cu") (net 16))
 (segment (start 81.5 70) (end 81.5 83.605) (width 0.2) (layer "F.Cu") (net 16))
 (segment (start 71.204025 111.469738) (end 71.204025 105.560757) (width 0.2) (layer "F.Cu") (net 16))
 (segment (start 81.307328 86.065) (end 66.507798 100.86453) (width 0.2) (layer "B.Cu") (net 16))
 (segment (start 83.96 86.065) (end 81.307328 86.065) (width 0.2) (layer "B.Cu") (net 16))
 (segment (start 89.04 72.54) (end 89.04 86.065) (width 0.2) (layer "F.Cu") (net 17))
 (segment (start 91.58 70) (end 89.04 72.54) (width 0.2) (layer "F.Cu") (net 17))
 (segment (start 85.349 87.89024) (end 85.349 85.58824) (width 0.2) (layer "B.Cu") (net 17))
 (segment (start 86.02324 84.914) (end 87.889 84.914) (width 0.2) (layer "B.Cu") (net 17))
 (segment (start 69.83471 103.40453) (end 85.349 87.89024) (width 0.2) (layer "B.Cu") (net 17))
 (segment (start 85.349 85.58824) (end 86.02324 84.914) (width 0.2) (layer "B.Cu") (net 17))
 (segment (start 87.889 84.914) (end 89.04 86.065) (width 0.2) (layer "B.Cu") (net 17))
 (segment (start 66.507798 103.40453) (end 69.83471 103.40453) (width 0.2) (layer "B.Cu") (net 17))
 (segment (start 80.340138 120.96991) (end 80.909369 121.539141) (width 0.2) (layer "F.Cu") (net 1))
 (segment (start 80.330942 112.502821) (end 80.340138 112.493625) (width 0.2) (layer "F.Cu") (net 1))
 (segment (start 80.340138 112.493625) (end 80.340138 120.96991) (width 0.2) (layer "F.Cu") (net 1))
 (segment (start 93.58 120.393376) (end 92.456848 121.516528) (width 0.2) (layer "F.Cu") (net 19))
 (segment (start 93.58 112.553862) (end 93.58 121.325216) (width 0.2) (layer "F.Cu") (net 19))
 (segment (start 93.58 121.325216) (end 93.399066 121.50615) (width 0.2) (layer "F.Cu") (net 19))
 (segment (start 87.269118 133.599059) (end 87.269118 132.963937) (width 0.2) (layer "F.Cu") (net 3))
 (segment (start 80.836603 140.031574) (end 87.269118 133.599059) (width 0.2) (layer "F.Cu") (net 3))
 (segment (start 58.887798 98.32453) (end 62.712328 94.5) (width 0.2) (layer "F.Cu") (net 23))
 (segment (start 62.712328 94.5) (end 68.84566 94.5) (width 0.2) (layer "F.Cu") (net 23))
 (segment (start 68.84566 94.5) (end 70.051822 95.706162) (width 0.2) (layer "F.Cu") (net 23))
 (segment (start 58.887798 95.78453) (end 56.52453 95.78453) (width 0.2) (layer "F.Cu") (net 10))
 (segment (start 56.52453 95.78453) (end 52 91.26) (width 0.2) (layer "F.Cu") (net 10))
 (segment (start 59.988798 107.04553) (end 59.988798 109.92353) (width 0.2) (layer "F.Cu") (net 26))
 (segment (start 58.887798 105.94453) (end 59.988798 107.04553) (width 0.2) (layer "F.Cu") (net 26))
 (segment (start 59.988798 109.92353) (end 58.887798 111.02453) (width 0.2) (layer "F.Cu") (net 26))
 (segment (start 54.399 104.37605) (end 54.399 102.601) (width 0.2) (layer "B.Cu") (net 26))
 (segment (start 55.96748 105.94453) (end 54.399 104.37605) (width 0.2) (layer "B.Cu") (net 26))
 (segment (start 54.399 102.601) (end 55.5 101.5) (width 0.2) (layer "B.Cu") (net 26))
 (segment (start 58.887798 105.94453) (end 55.96748 105.94453) (width 0.2) (layer "B.Cu") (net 26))
 (segment (start 58.887798 113.56453) (end 56.01547 113.56453) (width 0.2) (layer "F.Cu") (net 12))
 (segment (start 56.01547 113.56453) (end 55.5 114.08) (width 0.2) (layer "F.Cu") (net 12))
 (segment (start 87.899 105.15805) (end 87.899 100.871) (width 0.2) (layer "B.Cu") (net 12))
 (segment (start 87.899 100.871) (end 89 99.77) (width 0.2) (layer "B.Cu") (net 12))
 (segment (start 82.05705 111) (end 87.899 105.15805) (width 0.2) (layer "B.Cu") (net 12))
 (segment (start 59.988798 112.46353) (end 67.46353 112.46353) (width 0.2) (layer "B.Cu") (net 12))
 (segment (start 68.92706 111) (end 82.05705 111) (width 0.2) (layer "B.Cu") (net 12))
 (segment (start 67.46353 112.46353) (end 68.92706 111) (width 0.2) (layer "B.Cu") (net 12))
 (segment (start 58.887798 113.56453) (end 59.988798 112.46353) (width 0.2) (layer "B.Cu") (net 12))
 (segment (start 68.183268 100) (end 66.507798 98.32453) (width 0.2) (layer "F.Cu") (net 5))
 (segment (start 70.051822 100) (end 68.183268 100) (width 0.2) (layer "F.Cu") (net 5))
 (segment (start 66.507798 111.02453) (end 69.518965 108.013363) (width 0.2) (layer "F.Cu") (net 15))
 (segment (start 69.518965 108.013363) (end 70.103025 108.013363) (width 0.2) (layer "F.Cu") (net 15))
 (segment (start 65.406798 107.04553) (end 66.507798 105.94453) (width 0.2) (layer "F.Cu") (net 15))
 (segment (start 65.406798 109.92353) (end 65.406798 107.04553) (width 0.2) (layer "F.Cu") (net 15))
 (segment (start 66.507798 111.02453) (end 65.406798 109.92353) (width 0.2) (layer "F.Cu") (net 15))
 (segment (start 78.767001 106.912363) (end 78.767001 108.767001) (width 0.2) (layer "F.Cu") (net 20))
 (segment (start 78.767001 108.767001) (end 82.553862 112.553862) (width 0.2) (layer "F.Cu") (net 20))
 (segment (start 82.553862 112.553862) (end 83.42 112.553862) (width 0.2) (layer "F.Cu") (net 20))
 (segment (start 67.639168 95.78453) (end 78.767001 106.912363) (width 0.2) (layer "F.Cu") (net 20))
 (segment (start 66.507798 95.78453) (end 67.639168 95.78453) (width 0.2) (layer "F.Cu") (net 20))
 (segment (start 89 97.23) (end 89 94.69) (width 0.2) (layer "F.Cu") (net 13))
 (segment (start 90.101 98.331) (end 89 97.23) (width 0.2) (layer "F.Cu") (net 13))
 (segment (start 75.526714 133.004329) (end 90.101 118.430043) (width 0.2) (layer "F.Cu") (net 13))
 (segment (start 90.101 118.430043) (end 90.101 98.331) (width 0.2) (layer "F.Cu") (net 13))
 (segment (start 62.247323 133.004329) (end 75.526714 133.004329) (width 0.2) (layer "F.Cu") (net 13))
 (segment (start 93.66 105.27) (end 96.62 102.31) (width 0.2) (layer "F.Cu") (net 14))
 (segment (start 93.66 108) (end 93.66 105.27) (width 0.2) (layer "F.Cu") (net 14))
 (segment (start 87.295471 114.364529) (end 93.66 108) (width 0.2) (layer "B.Cu") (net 14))
 (segment (start 67.307797 114.364529) (end 87.295471 114.364529) (width 0.2) (layer "B.Cu") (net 14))
 (segment (start 66.507798 113.56453) (end 67.307797 114.364529) (width 0.2) (layer "B.Cu") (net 14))
 (segment (start 96.62 99.77) (end 96.62 97.23) (width 0.2) (layer "F.Cu") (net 2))
 (segment (start 98.229117 132.163938) (end 98.229117 101.379117) (width 0.2) (layer "F.Cu") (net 2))
 (segment (start 98.229117 101.379117) (end 96.62 99.77) (width 0.2) (layer "F.Cu") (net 2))
 (segment (start 97.429118 132.963937) (end 98.229117 132.163938) (width 0.2) (layer "F.Cu") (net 2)))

